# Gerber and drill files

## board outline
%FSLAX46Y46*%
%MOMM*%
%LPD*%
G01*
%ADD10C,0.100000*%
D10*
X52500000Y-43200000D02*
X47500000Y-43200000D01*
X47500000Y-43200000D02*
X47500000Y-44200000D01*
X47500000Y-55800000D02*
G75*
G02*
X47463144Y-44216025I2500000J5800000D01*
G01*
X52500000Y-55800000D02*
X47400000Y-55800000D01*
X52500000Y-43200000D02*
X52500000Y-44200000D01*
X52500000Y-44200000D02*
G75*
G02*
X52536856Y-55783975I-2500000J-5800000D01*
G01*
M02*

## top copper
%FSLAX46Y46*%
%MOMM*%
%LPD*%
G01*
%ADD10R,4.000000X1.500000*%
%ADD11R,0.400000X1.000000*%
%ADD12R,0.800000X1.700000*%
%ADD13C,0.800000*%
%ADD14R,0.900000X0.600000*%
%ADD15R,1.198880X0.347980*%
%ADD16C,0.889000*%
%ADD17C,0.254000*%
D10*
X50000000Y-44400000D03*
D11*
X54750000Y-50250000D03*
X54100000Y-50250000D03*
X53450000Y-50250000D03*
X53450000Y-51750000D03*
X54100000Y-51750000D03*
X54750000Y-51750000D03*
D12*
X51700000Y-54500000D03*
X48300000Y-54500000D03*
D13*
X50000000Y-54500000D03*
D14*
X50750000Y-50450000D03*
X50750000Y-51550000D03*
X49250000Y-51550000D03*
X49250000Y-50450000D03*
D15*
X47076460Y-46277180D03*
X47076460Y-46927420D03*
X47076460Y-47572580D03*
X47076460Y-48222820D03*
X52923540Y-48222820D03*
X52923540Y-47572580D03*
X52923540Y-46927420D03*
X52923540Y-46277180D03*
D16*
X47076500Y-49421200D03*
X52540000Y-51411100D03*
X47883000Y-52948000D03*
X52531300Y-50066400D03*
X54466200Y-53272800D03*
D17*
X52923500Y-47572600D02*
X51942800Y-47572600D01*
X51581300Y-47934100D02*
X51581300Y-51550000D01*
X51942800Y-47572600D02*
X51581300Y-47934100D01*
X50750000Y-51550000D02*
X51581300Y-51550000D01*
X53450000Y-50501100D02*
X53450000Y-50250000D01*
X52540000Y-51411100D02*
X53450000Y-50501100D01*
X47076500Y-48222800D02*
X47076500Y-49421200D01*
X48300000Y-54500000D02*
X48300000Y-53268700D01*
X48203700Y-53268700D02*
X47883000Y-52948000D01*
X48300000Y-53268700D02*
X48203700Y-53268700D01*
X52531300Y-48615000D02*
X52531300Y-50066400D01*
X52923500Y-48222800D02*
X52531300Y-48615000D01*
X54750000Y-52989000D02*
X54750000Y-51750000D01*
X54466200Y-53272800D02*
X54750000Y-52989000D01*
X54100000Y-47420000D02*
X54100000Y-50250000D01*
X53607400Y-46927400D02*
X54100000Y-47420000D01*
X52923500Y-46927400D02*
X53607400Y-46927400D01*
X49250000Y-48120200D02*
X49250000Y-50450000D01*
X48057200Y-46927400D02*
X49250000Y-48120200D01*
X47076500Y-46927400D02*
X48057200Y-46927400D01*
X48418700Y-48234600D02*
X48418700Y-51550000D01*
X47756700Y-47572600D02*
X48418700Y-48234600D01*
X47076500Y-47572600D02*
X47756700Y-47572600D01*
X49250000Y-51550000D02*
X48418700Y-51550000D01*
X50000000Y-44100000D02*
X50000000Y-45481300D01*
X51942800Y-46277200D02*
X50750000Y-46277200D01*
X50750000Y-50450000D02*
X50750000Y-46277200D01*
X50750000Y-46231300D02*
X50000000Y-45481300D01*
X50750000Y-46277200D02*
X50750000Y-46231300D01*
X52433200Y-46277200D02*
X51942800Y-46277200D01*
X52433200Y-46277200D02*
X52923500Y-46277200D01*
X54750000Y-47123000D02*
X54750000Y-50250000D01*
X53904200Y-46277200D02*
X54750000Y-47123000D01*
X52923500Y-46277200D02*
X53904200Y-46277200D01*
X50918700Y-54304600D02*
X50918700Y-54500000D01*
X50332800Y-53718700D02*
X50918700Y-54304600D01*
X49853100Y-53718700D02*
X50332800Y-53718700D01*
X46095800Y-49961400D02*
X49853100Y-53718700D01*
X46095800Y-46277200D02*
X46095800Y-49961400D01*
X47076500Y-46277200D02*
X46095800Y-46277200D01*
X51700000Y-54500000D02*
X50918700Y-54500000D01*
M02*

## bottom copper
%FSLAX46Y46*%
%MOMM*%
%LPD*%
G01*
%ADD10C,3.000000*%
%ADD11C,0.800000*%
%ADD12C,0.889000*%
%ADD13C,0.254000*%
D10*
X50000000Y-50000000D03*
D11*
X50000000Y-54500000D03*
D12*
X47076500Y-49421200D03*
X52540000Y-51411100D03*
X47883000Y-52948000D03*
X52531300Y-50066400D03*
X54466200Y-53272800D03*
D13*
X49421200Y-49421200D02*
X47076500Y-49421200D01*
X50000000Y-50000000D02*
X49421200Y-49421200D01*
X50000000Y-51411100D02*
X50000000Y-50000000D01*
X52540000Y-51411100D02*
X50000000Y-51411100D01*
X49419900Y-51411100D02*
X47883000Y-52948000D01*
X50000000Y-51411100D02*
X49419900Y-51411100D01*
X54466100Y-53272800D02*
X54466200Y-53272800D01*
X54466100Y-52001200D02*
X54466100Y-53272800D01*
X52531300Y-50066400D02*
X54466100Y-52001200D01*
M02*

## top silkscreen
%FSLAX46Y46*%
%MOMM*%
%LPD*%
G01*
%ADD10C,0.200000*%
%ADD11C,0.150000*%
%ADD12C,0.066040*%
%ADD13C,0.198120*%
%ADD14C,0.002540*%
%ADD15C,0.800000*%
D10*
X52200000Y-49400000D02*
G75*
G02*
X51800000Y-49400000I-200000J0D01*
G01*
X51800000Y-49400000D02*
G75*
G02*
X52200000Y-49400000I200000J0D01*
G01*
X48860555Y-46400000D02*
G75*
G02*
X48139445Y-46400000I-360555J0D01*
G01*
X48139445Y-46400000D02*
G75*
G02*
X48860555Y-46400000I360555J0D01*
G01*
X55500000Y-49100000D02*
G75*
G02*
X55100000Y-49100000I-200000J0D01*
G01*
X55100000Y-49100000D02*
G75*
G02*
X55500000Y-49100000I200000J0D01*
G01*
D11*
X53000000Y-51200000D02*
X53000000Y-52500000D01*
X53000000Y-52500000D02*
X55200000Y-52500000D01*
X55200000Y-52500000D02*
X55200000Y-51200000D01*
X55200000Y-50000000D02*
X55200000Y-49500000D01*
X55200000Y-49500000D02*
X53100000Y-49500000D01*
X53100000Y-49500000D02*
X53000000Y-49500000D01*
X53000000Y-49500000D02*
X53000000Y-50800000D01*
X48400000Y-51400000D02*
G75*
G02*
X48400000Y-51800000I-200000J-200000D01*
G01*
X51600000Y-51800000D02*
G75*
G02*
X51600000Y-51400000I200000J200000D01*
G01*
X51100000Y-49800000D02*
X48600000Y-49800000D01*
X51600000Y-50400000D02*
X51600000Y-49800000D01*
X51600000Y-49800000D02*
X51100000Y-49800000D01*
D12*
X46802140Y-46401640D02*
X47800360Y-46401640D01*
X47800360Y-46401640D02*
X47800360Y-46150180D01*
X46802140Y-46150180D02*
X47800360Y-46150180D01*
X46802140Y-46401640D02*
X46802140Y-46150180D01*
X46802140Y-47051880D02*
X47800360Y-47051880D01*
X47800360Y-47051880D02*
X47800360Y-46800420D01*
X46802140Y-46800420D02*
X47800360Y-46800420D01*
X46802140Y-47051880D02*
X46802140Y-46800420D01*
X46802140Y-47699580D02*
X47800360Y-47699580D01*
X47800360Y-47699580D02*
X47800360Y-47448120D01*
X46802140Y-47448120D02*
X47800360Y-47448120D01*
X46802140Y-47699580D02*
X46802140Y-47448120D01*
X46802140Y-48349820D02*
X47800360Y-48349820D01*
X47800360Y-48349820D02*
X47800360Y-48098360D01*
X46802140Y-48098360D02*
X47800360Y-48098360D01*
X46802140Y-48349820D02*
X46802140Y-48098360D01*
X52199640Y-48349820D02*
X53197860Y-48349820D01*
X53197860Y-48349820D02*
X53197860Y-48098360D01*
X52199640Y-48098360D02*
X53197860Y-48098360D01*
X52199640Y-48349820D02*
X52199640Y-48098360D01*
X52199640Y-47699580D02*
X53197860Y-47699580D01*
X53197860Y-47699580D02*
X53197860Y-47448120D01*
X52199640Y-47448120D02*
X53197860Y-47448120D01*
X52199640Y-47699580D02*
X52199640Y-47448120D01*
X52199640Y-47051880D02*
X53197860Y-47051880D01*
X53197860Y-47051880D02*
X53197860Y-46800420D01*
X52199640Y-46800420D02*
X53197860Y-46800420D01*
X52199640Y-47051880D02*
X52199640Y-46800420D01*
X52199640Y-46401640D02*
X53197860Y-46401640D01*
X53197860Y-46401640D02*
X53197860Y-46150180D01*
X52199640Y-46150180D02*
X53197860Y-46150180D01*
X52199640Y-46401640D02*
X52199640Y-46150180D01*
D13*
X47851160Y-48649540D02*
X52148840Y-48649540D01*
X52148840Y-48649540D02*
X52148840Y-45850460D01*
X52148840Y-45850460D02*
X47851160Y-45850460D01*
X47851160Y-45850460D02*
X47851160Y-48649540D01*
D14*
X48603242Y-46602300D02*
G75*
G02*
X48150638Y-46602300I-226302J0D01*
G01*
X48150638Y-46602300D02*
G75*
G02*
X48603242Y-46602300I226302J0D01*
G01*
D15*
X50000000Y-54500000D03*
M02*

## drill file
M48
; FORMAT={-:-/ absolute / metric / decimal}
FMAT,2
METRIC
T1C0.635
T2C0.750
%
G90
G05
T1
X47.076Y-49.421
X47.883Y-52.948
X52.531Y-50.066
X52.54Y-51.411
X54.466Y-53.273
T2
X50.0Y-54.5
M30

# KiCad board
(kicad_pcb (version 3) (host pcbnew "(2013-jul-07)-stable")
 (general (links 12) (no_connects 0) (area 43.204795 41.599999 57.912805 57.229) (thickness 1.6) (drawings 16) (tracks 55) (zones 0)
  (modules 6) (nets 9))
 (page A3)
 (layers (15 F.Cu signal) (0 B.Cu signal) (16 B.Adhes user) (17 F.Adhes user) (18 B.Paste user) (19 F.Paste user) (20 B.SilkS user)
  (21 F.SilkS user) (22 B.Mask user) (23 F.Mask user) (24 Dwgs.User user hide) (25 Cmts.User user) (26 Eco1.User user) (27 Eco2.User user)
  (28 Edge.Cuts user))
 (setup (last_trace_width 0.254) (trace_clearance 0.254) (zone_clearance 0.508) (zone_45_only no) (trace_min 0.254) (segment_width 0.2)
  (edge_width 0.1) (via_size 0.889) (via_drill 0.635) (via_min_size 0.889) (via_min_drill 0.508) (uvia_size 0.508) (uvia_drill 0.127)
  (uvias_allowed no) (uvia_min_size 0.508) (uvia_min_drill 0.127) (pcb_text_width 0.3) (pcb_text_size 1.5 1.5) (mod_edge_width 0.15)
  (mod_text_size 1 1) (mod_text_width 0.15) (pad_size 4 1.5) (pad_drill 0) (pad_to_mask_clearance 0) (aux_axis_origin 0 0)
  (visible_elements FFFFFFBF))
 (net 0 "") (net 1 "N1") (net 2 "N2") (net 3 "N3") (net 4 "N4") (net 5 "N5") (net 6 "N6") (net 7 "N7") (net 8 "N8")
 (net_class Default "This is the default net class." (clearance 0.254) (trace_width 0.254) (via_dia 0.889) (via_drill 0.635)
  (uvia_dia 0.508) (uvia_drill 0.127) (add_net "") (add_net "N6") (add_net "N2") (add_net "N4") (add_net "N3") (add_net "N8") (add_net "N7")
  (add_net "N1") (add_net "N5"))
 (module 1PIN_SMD (layer F.Cu) (at 50 44.4)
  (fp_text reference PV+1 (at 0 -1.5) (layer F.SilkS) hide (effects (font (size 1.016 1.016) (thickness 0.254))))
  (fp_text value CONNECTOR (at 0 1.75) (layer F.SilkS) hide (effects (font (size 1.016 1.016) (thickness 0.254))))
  (pad 1 smd rect (at 0 0) (size 4 1.5) (layers F.Cu F.Paste F.Mask) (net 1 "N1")))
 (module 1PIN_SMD (layer B.Cu) (at 50 50)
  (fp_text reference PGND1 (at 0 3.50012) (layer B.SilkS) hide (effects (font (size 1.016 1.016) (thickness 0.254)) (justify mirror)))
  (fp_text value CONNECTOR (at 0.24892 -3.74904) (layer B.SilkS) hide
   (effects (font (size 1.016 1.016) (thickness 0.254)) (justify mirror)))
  (pad 1 smd circle (at 0 0) (size 3 3) (layers B.Cu B.Paste B.Mask) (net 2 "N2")))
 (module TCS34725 (layer F.Cu) (at 54.1 51 90)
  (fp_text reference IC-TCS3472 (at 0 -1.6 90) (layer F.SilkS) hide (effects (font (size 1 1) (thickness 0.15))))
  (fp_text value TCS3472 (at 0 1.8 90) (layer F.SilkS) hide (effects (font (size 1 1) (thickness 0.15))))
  (fp_line (start -0.2 -1.1) (end -1.5 -1.1) (layer F.SilkS) (width 0.15))
  (fp_line (start -1.5 -1.1) (end -1.5 1.1) (layer F.SilkS) (width 0.15))
  (fp_line (start -1.5 1.1) (end -0.2 1.1) (layer F.SilkS) (width 0.15))
  (fp_line (start 1 1.1) (end 1.5 1.1) (layer F.SilkS) (width 0.15))
  (fp_line (start 1.5 1.1) (end 1.5 -1) (layer F.SilkS) (width 0.15))
  (fp_line (start 1.5 -1) (end 1.5 -1.1) (layer F.SilkS) (width 0.15))
  (fp_line (start 1.5 -1.1) (end 0.2 -1.1) (layer F.SilkS) (width 0.15))
  (pad 1 smd rect (at 0.75 0.65 90) (size 1 0.4) (layers F.Cu F.Paste F.Mask) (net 1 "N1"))
  (pad 2 smd rect (at 0.75 0 90) (size 1 0.4) (layers F.Cu F.Paste F.Mask) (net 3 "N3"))
  (pad 3 smd rect (at 0.75 -0.65 90) (size 1 0.4) (layers F.Cu F.Paste F.Mask) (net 2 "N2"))
  (pad 4 smd rect (at -0.75 -0.65 90) (size 1 0.4) (layers F.Cu F.Paste F.Mask))
  (pad 5 smd rect (at -0.75 0 90) (size 1 0.4) (layers F.Cu F.Paste F.Mask))
  (pad 6 smd rect (at -0.75 0.65 90) (size 1 0.4) (layers F.Cu F.Paste F.Mask) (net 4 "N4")))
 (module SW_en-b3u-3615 (layer F.Cu) (at 50 54.5 180)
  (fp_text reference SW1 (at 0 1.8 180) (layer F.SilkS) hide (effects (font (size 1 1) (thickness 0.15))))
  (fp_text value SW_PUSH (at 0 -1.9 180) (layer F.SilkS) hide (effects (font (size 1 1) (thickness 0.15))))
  (pad 1 smd rect (at -1.7 0 180) (size 0.8 1.7) (layers F.Cu F.Paste F.Mask) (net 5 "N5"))
  (pad 2 smd rect (at 1.7 0 180) (size 0.8 1.7) (layers F.Cu F.Paste F.Mask) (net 2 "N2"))
  (pad "" thru_hole circle (at 0 0 180) (size 0.8 0.8) (drill 0.75) (layers *.Cu *.Mask F.SilkS)))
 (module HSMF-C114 (layer F.Cu) (at 50 51 180)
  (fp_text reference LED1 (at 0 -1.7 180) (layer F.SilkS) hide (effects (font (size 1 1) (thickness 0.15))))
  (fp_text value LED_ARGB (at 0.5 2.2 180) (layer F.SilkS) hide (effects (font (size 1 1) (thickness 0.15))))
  (fp_arc (start 1.8 -0.6) (end 1.6 -0.4) (angle 90) (layer F.SilkS) (width 0.15))
  (fp_arc (start -1.8 -0.6) (end -1.6 -0.8) (angle 90) (layer F.SilkS) (width 0.15))
  (fp_line (start -1.1 1.2) (end 1.4 1.2) (layer F.SilkS) (width 0.15))
  (fp_line (start -1.6 0.6) (end -1.6 1.2) (layer F.SilkS) (width 0.15))
  (fp_line (start -1.6 1.2) (end -1.1 1.2) (layer F.SilkS) (width 0.15))
  (pad 1 smd rect (at -0.75 0.55 180) (size 0.9 0.6) (layers F.Cu F.Paste F.Mask) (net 1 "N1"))
  (pad 2 smd rect (at -0.75 -0.55 180) (size 0.9 0.6) (layers F.Cu F.Paste F.Mask) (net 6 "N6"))
  (pad 3 smd rect (at 0.75 -0.55 180) (size 0.9 0.6) (layers F.Cu F.Paste F.Mask) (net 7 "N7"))
  (pad 4 smd rect (at 0.75 0.55 180) (size 0.9 0.6) (layers F.Cu F.Paste F.Mask) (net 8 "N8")))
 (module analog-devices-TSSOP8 (layer F.Cu) (at 50 47.25)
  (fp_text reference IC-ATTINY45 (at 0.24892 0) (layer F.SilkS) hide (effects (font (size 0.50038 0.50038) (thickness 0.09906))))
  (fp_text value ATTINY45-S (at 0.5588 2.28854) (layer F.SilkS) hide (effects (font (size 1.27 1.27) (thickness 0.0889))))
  (fp_line (start -3.19786 -0.84836) (end -2.19964 -0.84836) (layer F.SilkS) (width 0.06604))
  (fp_line (start -2.19964 -0.84836) (end -2.19964 -1.09982) (layer F.SilkS) (width 0.06604))
  (fp_line (start -3.19786 -1.09982) (end -2.19964 -1.09982) (layer F.SilkS) (width 0.06604))
  (fp_line (start -3.19786 -0.84836) (end -3.19786 -1.09982) (layer F.SilkS) (width 0.06604))
  (fp_line (start -3.19786 -0.19812) (end -2.19964 -0.19812) (layer F.SilkS) (width 0.06604))
  (fp_line (start -2.19964 -0.19812) (end -2.19964 -0.44958) (layer F.SilkS) (width 0.06604))
  (fp_line (start -3.19786 -0.44958) (end -2.19964 -0.44958) (layer F.SilkS) (width 0.06604))
  (fp_line (start -3.19786 -0.19812) (end -3.19786 -0.44958) (layer F.SilkS) (width 0.06604))
  (fp_line (start -3.19786 0.44958) (end -2.19964 0.44958) (layer F.SilkS) (width 0.06604))
  (fp_line (start -2.19964 0.44958) (end -2.19964 0.19812) (layer F.SilkS) (width 0.06604))
  (fp_line (start -3.19786 0.19812) (end -2.19964 0.19812) (layer F.SilkS) (width 0.06604))
  (fp_line (start -3.19786 0.44958) (end -3.19786 0.19812) (layer F.SilkS) (width 0.06604))
  (fp_line (start -3.19786 1.09982) (end -2.19964 1.09982) (layer F.SilkS) (width 0.06604))
  (fp_line (start -2.19964 1.09982) (end -2.19964 0.84836) (layer F.SilkS) (width 0.06604))
  (fp_line (start -3.19786 0.84836) (end -2.19964 0.84836) (layer F.SilkS) (width 0.06604))
  (fp_line (start -3.19786 1.09982) (end -3.19786 0.84836) (layer F.SilkS) (width 0.06604))
  (fp_line (start 2.19964 1.09982) (end 3.19786 1.09982) (layer F.SilkS) (width 0.06604))
  (fp_line (start 3.19786 1.09982) (end 3.19786 0.84836) (layer F.SilkS) (width 0.06604))
  (fp_line (start 2.19964 0.84836) (end 3.19786 0.84836) (layer F.SilkS) (width 0.06604))
  (fp_line (start 2.19964 1.09982) (end 2.19964 0.84836) (layer F.SilkS) (width 0.06604))
  (fp_line (start 2.19964 0.44958) (end 3.19786 0.44958) (layer F.SilkS) (width 0.06604))
  (fp_line (start 3.19786 0.44958) (end 3.19786 0.19812) (layer F.SilkS) (width 0.06604))
  (fp_line (start 2.19964 0.19812) (end 3.19786 0.19812) (layer F.SilkS) (width 0.06604))
  (fp_line (start 2.19964 0.44958) (end 2.19964 0.19812) (layer F.SilkS) (width 0.06604))
  (fp_line (start 2.19964 -0.19812) (end 3.19786 -0.19812) (layer F.SilkS) (width 0.06604))
  (fp_line (start 3.19786 -0.19812) (end 3.19786 -0.44958) (layer F.SilkS) (width 0.06604))
  (fp_line (start 2.19964 -0.44958) (end 3.19786 -0.44958) (layer F.SilkS) (width 0.06604))
  (fp_line (start 2.19964 -0.19812) (end 2.19964 -0.44958) (layer F.SilkS) (width 0.06604))
  (fp_line (start 2.19964 -0.84836) (end 3.19786 -0.84836) (layer F.SilkS) (width 0.06604))
  (fp_line (start 3.19786 -0.84836) (end 3.19786 -1.09982) (layer F.SilkS) (width 0.06604))
  (fp_line (start 2.19964 -1.09982) (end 3.19786 -1.09982) (layer F.SilkS) (width 0.06604))
  (fp_line (start 2.19964 -0.84836) (end 2.19964 -1.09982) (layer F.SilkS) (width 0.06604))
  (fp_line (start -2.14884 1.39954) (end 2.14884 1.39954) (layer F.SilkS) (width 0.19812))
  (fp_line (start 2.14884 1.39954) (end 2.14884 -1.39954) (layer F.SilkS) (width 0.19812))
  (fp_line (start 2.14884 -1.39954) (end -2.14884 -1.39954) (layer F.SilkS) (width 0.19812))
  (fp_line (start -2.14884 -1.39954) (end -2.14884 1.39954) (layer F.SilkS) (width 0.19812))
  (fp_circle (center -1.62306 -0.6477) (end -1.78308 -0.80772) (layer F.SilkS) (width 0.00254))
  (pad 1 smd rect (at -2.92354 -0.97282) (size 1.19888 0.34798) (layers F.Cu F.Paste F.Mask) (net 5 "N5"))
  (pad 2 smd rect (at -2.92354 -0.32258) (size 1.19888 0.34798) (layers F.Cu F.Paste F.Mask) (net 8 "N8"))
  (pad 3 smd rect (at -2.92354 0.32258) (size 1.19888 0.34798) (layers F.Cu F.Paste F.Mask) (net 7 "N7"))
  (pad 4 smd rect (at -2.92354 0.97282) (size 1.19888 0.34798) (layers F.Cu F.Paste F.Mask) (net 2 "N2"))
  (pad 5 smd rect (at 2.92354 0.97282) (size 1.19888 0.34798) (layers F.Cu F.Paste F.Mask) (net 4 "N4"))
  (pad 6 smd rect (at 2.92354 0.32258) (size 1.19888 0.34798) (layers F.Cu F.Paste F.Mask) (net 6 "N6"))
  (pad 7 smd rect (at 2.92354 -0.32258) (size 1.19888 0.34798) (layers F.Cu F.Paste F.Mask) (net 3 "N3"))
  (pad 8 smd rect (at 2.92354 -0.97282) (size 1.19888 0.34798) (layers F.Cu F.Paste F.Mask) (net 1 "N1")))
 (gr_line (start 52.5 43.2) (end 47.5 43.2) (angle 90) (layer Edge.Cuts) (width 0.1))
 (gr_line (start 47.5 43.2) (end 47.5 44.2) (angle 90) (layer Edge.Cuts) (width 0.1))
 (gr_arc (start 50 50) (end 47.5 55.8) (angle 133) (layer Edge.Cuts) (width 0.1))
 (gr_line (start 52.5 55.8) (end 47.4 55.8) (angle 90) (layer Edge.Cuts) (width 0.1))
 (gr_line (start 52.5 43.2) (end 52.5 44.2) (angle 90) (layer Edge.Cuts) (width 0.1))
 (gr_arc (start 50 50) (end 52.5 44.2) (angle 133) (layer Edge.Cuts) (width 0.1))
 (gr_circle (center 52 49.4) (end 52 49.2) (layer F.SilkS) (width 0.2))
 (gr_circle (center 48.5 46.4) (end 48.8 46.6) (layer F.SilkS) (width 0.2))
 (gr_circle (center 55.3 49.1) (end 55.3 48.9) (layer F.SilkS) (width 0.2))
 (segment (start 52.9235 47.5726) (end 51.9428 47.5726) (width 0.254) (layer F.Cu) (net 6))
 (segment (start 51.5813 47.9341) (end 51.5813 51.55) (width 0.254) (layer F.Cu) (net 6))
 (segment (start 51.9428 47.5726) (end 51.5813 47.9341) (width 0.254) (layer F.Cu) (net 6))
 (segment (start 50.75 51.55) (end 51.5813 51.55) (width 0.254) (layer F.Cu) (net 6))
 (via (at 47.0765 49.4212) (size 0.889) (layers F.Cu B.Cu) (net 2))
 (via (at 52.54 51.4111) (size 0.889) (layers F.Cu B.Cu) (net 2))
 (via (at 47.883 52.948) (size 0.889) (layers F.Cu B.Cu) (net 2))
 (segment (start 53.45 50.5011) (end 53.45 50.25) (width 0.254) (layer F.Cu) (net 2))
 (segment (start 52.54 51.4111) (end 53.45 50.5011) (width 0.254) (layer F.Cu) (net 2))
 (segment (start 49.4212 49.4212) (end 47.0765 49.4212) (width 0.254) (layer B.Cu) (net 2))
 (segment (start 50 50) (end 49.4212 49.4212) (width 0.254) (layer B.Cu) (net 2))
 (segment (start 47.0765 48.2228) (end 47.0765 49.4212) (width 0.254) (layer F.Cu) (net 2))
 (segment (start 48.3 54.5) (end 48.3 53.2687) (width 0.254) (layer F.Cu) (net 2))
 (segment (start 48.2037 53.2687) (end 47.883 52.948) (width 0.254) (layer F.Cu) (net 2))
 (segment (start 48.3 53.2687) (end 48.2037 53.2687) (width 0.254) (layer F.Cu) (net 2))
 (segment (start 50 51.4111) (end 50 50) (width 0.254) (layer B.Cu) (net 2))
 (segment (start 52.54 51.4111) (end 50 51.4111) (width 0.254) (layer B.Cu) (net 2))
 (segment (start 49.4199 51.4111) (end 47.883 52.948) (width 0.254) (layer B.Cu) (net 2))
 (segment (start 50 51.4111) (end 49.4199 51.4111) (width 0.254) (layer B.Cu) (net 2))
 (via (at 52.5313 50.0664) (size 0.889) (layers F.Cu B.Cu) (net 4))
 (via (at 54.4662 53.2728) (size 0.889) (layers F.Cu B.Cu) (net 4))
 (segment (start 52.5313 48.615) (end 52.5313 50.0664) (width 0.254) (layer F.Cu) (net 4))
 (segment (start 52.9235 48.2228) (end 52.5313 48.615) (width 0.254) (layer F.Cu) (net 4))
 (segment (start 54.4661 53.2728) (end 54.4662 53.2728) (width 0.254) (layer B.Cu) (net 4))
 (segment (start 54.4661 52.0012) (end 54.4661 53.2728) (width 0.254) (layer B.Cu) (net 4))
 (segment (start 52.5313 50.0664) (end 54.4661 52.0012) (width 0.254) (layer B.Cu) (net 4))
 (segment (start 54.75 52.989) (end 54.75 51.75) (width 0.254) (layer F.Cu) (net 4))
 (segment (start 54.4662 53.2728) (end 54.75 52.989) (width 0.254) (layer F.Cu) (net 4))
 (segment (start 54.1 47.42) (end 54.1 50.25) (width 0.254) (layer F.Cu) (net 3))
 (segment (start 53.6074 46.9274) (end 54.1 47.42) (width 0.254) (layer F.Cu) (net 3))
 (segment (start 52.9235 46.9274) (end 53.6074 46.9274) (width 0.254) (layer F.Cu) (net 3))
 (segment (start 49.25 48.1202) (end 49.25 50.45) (width 0.254) (layer F.Cu) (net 8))
 (segment (start 48.0572 46.9274) (end 49.25 48.1202) (width 0.254) (layer F.Cu) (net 8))
 (segment (start 47.0765 46.9274) (end 48.0572 46.9274) (width 0.254) (layer F.Cu) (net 8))
 (segment (start 48.4187 48.2346) (end 48.4187 51.55) (width 0.254) (layer F.Cu) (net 7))
 (segment (start 47.7567 47.5726) (end 48.4187 48.2346) (width 0.254) (layer F.Cu) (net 7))
 (segment (start 47.0765 47.5726) (end 47.7567 47.5726) (width 0.254) (layer F.Cu) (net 7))
 (segment (start 49.25 51.55) (end 48.4187 51.55) (width 0.254) (layer F.Cu) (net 7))
 (segment (start 50 44.1) (end 50 45.4813) (width 0.254) (layer F.Cu) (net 1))
 (segment (start 51.9428 46.2772) (end 50.75 46.2772) (width 0.254) (layer F.Cu) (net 1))
 (segment (start 50.75 50.45) (end 50.75 46.2772) (width 0.254) (layer F.Cu) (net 1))
 (segment (start 50.75 46.2313) (end 50 45.4813) (width 0.254) (layer F.Cu) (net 1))
 (segment (start 50.75 46.2772) (end 50.75 46.2313) (width 0.254) (layer F.Cu) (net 1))
 (segment (start 52.4332 46.2772) (end 51.9428 46.2772) (width 0.254) (layer F.Cu) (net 1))
 (segment (start 52.4332 46.2772) (end 52.9235 46.2772) (width 0.254) (layer F.Cu) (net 1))
 (segment (start 54.75 47.123) (end 54.75 50.25) (width 0.254) (layer F.Cu) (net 1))
 (segment (start 53.9042 46.2772) (end 54.75 47.123) (width 0.254) (layer F.Cu) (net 1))
 (segment (start 52.9235 46.2772) (end 53.9042 46.2772) (width 0.254) (layer F.Cu) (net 1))
 (segment (start 50.9187 54.3046) (end 50.9187 54.5) (width 0.254) (layer F.Cu) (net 5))
 (segment (start 50.3328 53.7187) (end 50.9187 54.3046) (width 0.254) (layer F.Cu) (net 5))
 (segment (start 49.8531 53.7187) (end 50.3328 53.7187) (width 0.254) (layer F.Cu) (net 5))
 (segment (start 46.0958 49.9614) (end 49.8531 53.7187) (width 0.254) (layer F.Cu) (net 5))
 (segment (start 46.0958 46.2772) (end 46.0958 49.9614) (width 0.254) (layer F.Cu) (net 5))
 (segment (start 47.0765 46.2772) (end 46.0958 46.2772) (width 0.254) (layer F.Cu) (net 5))
 (segment (start 51.7 54.5) (end 50.9187 54.5) (width 0.254) (layer F.Cu) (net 5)))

